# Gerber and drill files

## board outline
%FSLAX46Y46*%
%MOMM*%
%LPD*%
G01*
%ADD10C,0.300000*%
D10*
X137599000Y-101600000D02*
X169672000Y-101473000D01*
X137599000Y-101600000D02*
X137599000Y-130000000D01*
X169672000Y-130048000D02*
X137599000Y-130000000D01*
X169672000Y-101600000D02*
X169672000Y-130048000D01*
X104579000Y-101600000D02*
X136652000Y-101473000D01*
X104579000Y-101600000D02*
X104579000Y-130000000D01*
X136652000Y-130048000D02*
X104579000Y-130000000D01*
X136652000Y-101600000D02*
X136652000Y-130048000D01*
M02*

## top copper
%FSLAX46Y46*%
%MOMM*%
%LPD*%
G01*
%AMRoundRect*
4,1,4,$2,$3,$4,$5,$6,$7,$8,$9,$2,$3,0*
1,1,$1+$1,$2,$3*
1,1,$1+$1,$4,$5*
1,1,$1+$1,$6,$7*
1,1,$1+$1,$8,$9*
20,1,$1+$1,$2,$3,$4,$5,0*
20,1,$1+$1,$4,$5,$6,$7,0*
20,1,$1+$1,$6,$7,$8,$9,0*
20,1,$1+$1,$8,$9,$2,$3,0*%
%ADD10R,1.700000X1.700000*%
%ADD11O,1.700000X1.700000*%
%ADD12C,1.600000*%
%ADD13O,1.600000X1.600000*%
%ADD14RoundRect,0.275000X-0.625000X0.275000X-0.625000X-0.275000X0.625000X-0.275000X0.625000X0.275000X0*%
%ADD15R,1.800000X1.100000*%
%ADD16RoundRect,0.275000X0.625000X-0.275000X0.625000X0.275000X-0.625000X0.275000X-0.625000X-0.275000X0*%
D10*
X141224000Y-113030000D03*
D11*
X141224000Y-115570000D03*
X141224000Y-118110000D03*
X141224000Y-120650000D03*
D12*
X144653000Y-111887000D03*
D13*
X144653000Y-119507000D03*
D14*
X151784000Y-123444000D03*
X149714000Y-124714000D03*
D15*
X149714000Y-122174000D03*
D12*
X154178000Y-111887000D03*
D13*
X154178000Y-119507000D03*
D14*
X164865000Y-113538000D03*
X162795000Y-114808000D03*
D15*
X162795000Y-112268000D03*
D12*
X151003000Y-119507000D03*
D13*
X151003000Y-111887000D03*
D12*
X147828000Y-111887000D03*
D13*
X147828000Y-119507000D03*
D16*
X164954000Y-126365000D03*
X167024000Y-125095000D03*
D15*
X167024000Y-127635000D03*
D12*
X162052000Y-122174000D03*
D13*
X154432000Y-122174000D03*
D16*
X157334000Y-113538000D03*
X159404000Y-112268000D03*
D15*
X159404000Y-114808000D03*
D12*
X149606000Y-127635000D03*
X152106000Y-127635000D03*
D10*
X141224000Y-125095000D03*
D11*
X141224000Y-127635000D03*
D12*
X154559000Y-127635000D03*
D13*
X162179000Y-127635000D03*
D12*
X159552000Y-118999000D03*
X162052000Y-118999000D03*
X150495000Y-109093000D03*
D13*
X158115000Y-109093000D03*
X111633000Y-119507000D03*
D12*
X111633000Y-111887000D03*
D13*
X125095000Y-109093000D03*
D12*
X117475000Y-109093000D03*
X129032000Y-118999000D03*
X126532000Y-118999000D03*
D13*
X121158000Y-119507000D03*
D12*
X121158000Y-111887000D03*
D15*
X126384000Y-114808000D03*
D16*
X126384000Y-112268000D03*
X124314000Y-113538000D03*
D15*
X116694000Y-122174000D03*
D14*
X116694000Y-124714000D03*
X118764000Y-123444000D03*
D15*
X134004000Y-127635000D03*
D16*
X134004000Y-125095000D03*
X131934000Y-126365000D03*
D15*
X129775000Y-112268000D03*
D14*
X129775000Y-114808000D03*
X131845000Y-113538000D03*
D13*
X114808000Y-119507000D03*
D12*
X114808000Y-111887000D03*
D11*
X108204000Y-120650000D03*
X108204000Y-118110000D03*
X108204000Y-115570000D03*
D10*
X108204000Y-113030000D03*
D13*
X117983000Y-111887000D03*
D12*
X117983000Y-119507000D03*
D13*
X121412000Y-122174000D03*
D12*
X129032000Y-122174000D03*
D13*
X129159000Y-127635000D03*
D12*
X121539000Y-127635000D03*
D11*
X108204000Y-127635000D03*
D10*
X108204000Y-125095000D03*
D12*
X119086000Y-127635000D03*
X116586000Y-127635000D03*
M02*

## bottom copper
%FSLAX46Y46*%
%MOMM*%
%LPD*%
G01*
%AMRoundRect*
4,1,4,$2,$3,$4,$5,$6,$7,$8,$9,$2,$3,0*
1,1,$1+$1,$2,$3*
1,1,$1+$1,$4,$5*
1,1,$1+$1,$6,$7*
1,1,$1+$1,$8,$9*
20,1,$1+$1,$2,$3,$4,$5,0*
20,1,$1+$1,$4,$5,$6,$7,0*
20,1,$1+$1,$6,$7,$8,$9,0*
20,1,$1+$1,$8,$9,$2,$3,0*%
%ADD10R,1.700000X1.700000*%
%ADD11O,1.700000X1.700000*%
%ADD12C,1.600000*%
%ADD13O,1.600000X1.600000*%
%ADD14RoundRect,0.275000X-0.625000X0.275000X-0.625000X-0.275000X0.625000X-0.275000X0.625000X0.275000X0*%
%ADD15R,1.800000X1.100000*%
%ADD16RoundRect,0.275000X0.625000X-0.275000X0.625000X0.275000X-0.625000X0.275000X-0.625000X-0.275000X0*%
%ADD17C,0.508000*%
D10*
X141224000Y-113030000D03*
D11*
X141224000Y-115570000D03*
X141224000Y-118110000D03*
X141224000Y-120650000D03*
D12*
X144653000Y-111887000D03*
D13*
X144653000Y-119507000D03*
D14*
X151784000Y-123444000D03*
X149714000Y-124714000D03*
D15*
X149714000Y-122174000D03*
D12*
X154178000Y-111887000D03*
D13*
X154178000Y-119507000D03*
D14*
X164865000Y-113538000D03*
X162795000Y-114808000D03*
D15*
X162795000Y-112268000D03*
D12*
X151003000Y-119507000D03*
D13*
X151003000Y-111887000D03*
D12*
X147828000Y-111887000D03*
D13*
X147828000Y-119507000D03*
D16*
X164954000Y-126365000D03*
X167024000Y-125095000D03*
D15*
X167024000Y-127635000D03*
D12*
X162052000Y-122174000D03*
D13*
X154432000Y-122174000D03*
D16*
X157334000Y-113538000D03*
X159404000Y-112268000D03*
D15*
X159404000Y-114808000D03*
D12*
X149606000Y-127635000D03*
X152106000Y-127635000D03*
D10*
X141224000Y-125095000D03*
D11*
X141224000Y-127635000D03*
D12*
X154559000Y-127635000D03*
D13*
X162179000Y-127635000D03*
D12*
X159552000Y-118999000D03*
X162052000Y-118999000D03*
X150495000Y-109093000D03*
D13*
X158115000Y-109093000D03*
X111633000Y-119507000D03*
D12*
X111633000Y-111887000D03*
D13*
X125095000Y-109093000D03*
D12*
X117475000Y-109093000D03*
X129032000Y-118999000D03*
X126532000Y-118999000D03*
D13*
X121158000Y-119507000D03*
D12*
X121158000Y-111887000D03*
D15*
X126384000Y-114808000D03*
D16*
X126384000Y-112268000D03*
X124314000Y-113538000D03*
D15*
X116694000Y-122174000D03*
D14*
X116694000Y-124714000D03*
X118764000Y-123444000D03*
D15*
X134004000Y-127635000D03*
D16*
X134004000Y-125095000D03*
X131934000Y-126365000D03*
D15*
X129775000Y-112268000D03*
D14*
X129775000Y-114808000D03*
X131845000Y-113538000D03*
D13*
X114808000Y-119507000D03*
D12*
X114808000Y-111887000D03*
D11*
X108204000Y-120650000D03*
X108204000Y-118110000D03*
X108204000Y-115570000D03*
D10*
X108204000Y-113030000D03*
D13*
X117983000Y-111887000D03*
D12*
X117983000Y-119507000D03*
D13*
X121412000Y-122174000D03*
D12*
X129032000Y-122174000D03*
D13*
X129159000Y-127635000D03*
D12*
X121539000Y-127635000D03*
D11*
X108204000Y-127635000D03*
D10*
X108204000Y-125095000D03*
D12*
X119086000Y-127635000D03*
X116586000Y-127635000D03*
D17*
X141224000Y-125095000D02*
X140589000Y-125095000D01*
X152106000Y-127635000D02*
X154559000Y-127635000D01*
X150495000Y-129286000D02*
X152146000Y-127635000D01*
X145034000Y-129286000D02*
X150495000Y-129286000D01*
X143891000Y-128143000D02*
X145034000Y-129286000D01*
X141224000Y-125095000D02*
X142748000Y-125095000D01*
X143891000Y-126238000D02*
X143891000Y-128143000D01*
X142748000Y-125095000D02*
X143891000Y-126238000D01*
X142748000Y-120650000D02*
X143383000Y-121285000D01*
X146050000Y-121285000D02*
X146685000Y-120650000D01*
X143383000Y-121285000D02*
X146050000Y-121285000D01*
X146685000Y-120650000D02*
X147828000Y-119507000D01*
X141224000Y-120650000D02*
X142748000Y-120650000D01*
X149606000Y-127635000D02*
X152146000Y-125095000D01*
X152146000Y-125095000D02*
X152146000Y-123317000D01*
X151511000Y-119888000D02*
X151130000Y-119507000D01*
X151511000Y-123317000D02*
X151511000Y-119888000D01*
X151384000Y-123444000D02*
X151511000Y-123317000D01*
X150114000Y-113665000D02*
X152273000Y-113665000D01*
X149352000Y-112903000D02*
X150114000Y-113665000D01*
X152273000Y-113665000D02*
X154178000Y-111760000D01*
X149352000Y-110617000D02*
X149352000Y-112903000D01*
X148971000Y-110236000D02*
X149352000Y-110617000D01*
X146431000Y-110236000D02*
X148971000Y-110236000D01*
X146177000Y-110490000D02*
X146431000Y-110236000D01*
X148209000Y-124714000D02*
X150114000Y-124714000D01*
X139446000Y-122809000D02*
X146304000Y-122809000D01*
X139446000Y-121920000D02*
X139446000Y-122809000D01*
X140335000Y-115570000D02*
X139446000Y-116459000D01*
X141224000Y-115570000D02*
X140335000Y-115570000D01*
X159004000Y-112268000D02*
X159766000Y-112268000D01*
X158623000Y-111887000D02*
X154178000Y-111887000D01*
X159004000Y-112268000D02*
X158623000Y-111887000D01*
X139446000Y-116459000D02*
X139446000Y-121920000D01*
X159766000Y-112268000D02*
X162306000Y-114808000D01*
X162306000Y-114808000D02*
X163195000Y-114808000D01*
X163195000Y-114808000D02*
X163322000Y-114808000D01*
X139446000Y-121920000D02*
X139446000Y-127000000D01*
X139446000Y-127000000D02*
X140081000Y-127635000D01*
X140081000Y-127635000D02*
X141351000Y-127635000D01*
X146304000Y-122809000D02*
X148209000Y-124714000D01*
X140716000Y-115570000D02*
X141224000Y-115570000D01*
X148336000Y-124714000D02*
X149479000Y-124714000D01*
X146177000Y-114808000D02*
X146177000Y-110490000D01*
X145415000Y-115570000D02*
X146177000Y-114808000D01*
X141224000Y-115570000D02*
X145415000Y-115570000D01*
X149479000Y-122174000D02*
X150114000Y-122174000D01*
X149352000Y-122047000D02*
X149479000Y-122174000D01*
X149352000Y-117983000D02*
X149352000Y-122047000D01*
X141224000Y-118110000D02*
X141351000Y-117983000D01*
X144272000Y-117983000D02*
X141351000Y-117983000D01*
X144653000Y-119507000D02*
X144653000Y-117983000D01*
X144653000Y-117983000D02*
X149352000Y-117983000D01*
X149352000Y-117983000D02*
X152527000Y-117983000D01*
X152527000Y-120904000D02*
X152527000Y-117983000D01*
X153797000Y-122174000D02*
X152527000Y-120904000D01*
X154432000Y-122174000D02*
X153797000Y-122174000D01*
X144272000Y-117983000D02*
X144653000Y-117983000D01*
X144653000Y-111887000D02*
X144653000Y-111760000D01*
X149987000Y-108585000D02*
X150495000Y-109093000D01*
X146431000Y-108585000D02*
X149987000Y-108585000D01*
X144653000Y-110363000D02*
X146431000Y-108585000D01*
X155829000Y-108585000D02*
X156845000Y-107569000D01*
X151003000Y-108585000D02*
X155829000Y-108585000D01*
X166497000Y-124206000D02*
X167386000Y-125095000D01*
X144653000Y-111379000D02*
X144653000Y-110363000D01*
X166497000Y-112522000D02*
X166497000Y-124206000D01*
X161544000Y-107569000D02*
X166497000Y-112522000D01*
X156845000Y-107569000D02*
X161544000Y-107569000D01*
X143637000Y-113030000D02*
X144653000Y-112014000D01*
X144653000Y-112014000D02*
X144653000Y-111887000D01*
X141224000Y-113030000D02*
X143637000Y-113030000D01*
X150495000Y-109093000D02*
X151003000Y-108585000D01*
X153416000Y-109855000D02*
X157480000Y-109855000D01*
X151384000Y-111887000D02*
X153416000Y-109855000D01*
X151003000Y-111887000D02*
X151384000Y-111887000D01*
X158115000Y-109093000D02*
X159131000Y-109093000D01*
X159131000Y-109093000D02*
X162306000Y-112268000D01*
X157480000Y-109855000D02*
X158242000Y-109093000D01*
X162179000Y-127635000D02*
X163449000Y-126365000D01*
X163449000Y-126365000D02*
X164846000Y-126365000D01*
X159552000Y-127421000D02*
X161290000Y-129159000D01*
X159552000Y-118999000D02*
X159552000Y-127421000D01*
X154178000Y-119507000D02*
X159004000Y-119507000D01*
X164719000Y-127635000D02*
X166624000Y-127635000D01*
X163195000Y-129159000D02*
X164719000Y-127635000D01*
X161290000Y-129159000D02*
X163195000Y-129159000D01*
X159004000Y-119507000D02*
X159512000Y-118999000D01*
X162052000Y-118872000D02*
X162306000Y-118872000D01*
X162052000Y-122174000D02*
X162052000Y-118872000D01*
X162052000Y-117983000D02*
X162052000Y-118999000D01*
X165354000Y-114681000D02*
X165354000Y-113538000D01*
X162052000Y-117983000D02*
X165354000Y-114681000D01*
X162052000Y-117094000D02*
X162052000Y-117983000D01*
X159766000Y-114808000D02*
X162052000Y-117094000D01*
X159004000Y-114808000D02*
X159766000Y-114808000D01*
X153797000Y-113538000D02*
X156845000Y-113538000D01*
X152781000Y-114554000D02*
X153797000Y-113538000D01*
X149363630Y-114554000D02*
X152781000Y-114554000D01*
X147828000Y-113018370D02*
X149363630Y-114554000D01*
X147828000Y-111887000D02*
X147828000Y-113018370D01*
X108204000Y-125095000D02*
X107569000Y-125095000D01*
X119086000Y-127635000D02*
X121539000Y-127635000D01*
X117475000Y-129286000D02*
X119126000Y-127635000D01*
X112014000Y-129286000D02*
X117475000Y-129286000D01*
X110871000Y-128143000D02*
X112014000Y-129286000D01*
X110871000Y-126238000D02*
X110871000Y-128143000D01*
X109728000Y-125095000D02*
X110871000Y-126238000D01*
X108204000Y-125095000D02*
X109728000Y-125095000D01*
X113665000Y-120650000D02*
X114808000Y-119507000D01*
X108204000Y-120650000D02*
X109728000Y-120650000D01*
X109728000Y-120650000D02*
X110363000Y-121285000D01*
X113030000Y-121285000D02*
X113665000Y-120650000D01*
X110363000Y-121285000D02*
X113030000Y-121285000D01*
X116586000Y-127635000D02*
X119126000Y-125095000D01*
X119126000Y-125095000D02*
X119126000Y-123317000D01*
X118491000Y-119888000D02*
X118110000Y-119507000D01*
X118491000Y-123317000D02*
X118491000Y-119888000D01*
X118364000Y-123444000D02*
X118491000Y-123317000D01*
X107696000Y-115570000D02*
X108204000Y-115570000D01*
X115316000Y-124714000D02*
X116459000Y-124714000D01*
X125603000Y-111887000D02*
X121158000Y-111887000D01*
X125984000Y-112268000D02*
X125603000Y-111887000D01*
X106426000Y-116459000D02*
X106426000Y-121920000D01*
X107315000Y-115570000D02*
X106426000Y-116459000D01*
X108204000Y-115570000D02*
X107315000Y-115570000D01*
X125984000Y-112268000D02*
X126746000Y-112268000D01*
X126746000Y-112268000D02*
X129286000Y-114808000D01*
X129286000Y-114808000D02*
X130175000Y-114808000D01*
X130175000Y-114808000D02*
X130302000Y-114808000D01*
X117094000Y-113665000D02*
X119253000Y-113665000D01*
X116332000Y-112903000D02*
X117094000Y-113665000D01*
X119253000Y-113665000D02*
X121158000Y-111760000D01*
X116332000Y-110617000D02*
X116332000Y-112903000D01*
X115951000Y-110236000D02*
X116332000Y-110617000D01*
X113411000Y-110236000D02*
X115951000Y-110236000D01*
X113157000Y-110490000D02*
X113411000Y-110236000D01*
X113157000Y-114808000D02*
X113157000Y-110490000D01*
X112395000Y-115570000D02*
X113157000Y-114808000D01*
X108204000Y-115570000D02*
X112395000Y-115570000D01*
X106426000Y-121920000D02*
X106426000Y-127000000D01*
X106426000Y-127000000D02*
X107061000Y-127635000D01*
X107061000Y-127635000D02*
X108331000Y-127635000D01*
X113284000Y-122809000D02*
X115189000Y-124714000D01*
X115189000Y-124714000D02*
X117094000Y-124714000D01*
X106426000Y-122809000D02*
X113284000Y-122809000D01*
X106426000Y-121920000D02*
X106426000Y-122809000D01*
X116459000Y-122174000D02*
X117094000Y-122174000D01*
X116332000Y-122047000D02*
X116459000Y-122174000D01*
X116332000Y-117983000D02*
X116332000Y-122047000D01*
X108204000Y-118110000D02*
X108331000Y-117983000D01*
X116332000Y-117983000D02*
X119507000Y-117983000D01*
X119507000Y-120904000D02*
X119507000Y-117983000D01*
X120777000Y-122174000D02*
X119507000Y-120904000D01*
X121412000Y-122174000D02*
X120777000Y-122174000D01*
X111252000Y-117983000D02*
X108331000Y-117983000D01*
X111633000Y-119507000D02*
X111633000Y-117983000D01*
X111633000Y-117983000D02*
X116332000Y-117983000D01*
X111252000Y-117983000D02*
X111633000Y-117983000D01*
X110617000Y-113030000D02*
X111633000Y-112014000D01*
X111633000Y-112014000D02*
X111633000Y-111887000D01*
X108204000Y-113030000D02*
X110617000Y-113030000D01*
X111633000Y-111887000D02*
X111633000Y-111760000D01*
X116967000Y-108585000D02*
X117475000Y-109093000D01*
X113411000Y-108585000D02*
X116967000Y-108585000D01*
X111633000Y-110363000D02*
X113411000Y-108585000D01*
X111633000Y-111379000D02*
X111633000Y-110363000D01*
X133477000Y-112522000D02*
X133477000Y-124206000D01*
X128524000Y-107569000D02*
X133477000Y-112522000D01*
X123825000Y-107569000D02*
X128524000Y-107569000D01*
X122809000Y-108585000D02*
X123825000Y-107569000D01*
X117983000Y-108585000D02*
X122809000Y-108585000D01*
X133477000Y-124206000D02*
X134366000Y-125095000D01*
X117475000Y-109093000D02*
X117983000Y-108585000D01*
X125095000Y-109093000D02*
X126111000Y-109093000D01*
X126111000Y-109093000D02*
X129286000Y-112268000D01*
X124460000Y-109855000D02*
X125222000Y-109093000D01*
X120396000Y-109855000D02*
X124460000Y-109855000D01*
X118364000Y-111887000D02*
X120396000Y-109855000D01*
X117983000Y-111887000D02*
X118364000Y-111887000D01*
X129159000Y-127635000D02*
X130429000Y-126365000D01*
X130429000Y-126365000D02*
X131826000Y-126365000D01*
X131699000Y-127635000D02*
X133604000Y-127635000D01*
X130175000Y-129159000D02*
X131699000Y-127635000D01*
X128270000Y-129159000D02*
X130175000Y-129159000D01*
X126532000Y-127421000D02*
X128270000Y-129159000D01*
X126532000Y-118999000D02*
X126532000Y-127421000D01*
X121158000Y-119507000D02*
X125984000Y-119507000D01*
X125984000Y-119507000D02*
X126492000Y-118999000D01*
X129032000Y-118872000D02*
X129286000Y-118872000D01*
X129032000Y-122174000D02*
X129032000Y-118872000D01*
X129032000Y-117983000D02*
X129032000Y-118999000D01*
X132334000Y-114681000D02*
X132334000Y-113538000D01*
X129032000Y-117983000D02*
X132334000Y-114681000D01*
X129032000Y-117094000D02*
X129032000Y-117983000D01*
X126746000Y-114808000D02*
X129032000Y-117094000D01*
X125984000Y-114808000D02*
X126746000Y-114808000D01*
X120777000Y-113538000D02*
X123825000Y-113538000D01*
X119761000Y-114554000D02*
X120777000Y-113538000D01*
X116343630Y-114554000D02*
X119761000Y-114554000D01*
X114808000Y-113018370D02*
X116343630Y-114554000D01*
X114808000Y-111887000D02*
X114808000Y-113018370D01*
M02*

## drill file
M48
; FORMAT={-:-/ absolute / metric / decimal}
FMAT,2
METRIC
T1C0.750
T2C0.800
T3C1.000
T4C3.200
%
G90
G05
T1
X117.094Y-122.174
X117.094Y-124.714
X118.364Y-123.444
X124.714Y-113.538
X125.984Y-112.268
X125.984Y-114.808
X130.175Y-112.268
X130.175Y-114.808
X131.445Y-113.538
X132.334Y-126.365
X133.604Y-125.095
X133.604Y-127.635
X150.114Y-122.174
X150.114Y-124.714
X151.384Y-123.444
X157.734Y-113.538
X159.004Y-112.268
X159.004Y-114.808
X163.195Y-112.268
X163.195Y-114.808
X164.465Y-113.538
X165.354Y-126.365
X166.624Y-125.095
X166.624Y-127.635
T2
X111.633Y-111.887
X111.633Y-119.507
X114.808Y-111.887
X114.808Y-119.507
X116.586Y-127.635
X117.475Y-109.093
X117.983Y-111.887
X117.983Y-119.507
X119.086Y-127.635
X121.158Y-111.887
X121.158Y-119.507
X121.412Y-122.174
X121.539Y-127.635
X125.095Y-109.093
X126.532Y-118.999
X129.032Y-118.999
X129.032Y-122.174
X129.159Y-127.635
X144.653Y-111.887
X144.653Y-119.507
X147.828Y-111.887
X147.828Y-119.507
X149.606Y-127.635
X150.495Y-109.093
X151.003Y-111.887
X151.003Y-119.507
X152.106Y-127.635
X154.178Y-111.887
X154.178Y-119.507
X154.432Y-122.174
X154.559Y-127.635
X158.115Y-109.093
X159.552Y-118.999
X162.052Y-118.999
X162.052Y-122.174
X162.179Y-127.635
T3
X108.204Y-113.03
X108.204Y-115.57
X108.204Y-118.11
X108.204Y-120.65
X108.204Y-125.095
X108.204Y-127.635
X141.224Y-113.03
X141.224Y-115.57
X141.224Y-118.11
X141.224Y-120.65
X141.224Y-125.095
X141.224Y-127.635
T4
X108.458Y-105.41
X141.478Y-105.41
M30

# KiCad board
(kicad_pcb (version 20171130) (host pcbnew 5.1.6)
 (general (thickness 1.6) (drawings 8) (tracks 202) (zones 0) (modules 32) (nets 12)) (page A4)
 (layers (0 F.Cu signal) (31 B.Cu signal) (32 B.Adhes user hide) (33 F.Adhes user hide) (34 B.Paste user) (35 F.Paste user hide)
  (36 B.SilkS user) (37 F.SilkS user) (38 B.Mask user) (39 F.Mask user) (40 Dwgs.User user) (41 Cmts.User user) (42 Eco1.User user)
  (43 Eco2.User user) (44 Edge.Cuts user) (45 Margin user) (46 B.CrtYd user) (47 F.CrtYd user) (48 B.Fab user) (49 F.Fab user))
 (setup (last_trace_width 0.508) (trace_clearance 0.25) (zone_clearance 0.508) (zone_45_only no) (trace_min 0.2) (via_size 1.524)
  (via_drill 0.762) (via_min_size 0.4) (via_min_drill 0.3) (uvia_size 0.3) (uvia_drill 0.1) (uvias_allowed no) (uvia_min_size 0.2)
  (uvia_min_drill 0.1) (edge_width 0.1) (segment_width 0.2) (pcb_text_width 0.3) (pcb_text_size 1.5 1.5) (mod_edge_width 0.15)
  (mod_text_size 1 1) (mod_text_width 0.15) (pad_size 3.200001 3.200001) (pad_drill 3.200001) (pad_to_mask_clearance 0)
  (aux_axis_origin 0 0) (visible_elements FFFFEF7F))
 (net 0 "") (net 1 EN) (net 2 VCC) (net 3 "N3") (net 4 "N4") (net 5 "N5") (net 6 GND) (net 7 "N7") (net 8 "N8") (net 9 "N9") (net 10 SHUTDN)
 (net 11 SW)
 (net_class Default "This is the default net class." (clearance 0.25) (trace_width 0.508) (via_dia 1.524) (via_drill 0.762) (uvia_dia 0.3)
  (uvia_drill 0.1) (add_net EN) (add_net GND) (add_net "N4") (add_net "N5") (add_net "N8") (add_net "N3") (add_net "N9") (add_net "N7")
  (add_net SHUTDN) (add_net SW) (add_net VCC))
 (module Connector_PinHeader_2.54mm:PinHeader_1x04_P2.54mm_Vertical (layer F.Cu) (at 141.224 113.03)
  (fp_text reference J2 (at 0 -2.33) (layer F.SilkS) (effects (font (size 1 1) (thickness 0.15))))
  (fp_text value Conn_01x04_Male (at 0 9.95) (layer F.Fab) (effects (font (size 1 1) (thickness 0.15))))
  (pad 1 thru_hole rect (at 0 0) (size 1.7 1.7) (drill 1) (layers *.Cu *.Mask))
  (pad 2 thru_hole oval (at 0 2.54) (size 1.7 1.7) (drill 1) (layers *.Cu *.Mask))
  (pad 3 thru_hole oval (at 0 5.08) (size 1.7 1.7) (drill 1) (layers *.Cu *.Mask))
  (pad 4 thru_hole oval (at 0 7.62) (size 1.7 1.7) (drill 1) (layers *.Cu *.Mask)))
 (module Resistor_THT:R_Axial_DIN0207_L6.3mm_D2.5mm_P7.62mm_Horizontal (layer F.Cu) (at 144.653 111.887 270)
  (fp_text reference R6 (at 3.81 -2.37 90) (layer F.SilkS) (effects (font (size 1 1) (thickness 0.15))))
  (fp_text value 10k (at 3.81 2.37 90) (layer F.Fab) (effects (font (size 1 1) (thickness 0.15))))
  (pad 1 thru_hole circle (at 0 0 270) (size 1.6 1.6) (drill 0.8) (layers *.Cu *.Mask))
  (pad 2 thru_hole oval (at 7.62 0 270) (size 1.6 1.6) (drill 0.8) (layers *.Cu *.Mask)))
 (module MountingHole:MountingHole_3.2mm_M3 (layer F.Cu) (at 141.478 105.41)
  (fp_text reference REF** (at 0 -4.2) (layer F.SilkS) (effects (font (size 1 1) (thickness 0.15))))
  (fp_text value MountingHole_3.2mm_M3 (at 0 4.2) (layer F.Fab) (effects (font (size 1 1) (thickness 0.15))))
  (pad "" np_thru_hole circle (at 0 0) (size 3.200001 3.200001) (drill 3.200001) (layers *.Cu *.Mask)))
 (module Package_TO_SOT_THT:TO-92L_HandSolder (layer F.Cu) (at 150.114 122.174 270)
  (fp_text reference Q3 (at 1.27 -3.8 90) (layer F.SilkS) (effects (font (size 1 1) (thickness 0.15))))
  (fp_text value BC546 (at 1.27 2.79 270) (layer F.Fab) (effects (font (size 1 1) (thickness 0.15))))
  (pad 2 thru_hole roundrect (at 1.27 -1.27 270) (size 1.1 1.8) (drill 0.75 (offset 0 -0.4)) (layers *.Cu *.Mask) (roundrect_rratio 0.25))
  (pad 3 thru_hole roundrect (at 2.54 0 270) (size 1.1 1.8) (drill 0.75 (offset 0 0.4)) (layers *.Cu *.Mask) (roundrect_rratio 0.25))
  (pad 1 thru_hole rect (at 0 0 270) (size 1.1 1.8) (drill 0.75 (offset 0 0.4)) (layers *.Cu *.Mask)))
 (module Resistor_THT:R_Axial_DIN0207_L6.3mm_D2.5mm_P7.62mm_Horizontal (layer F.Cu) (at 154.178 111.887 270)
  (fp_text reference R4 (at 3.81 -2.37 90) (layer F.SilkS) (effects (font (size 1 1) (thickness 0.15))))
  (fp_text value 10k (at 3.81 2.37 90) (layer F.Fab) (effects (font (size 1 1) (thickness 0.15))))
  (pad 1 thru_hole circle (at 0 0 270) (size 1.6 1.6) (drill 0.8) (layers *.Cu *.Mask))
  (pad 2 thru_hole oval (at 7.62 0 270) (size 1.6 1.6) (drill 0.8) (layers *.Cu *.Mask)))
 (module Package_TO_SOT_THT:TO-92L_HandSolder (layer F.Cu) (at 163.195 112.268 270)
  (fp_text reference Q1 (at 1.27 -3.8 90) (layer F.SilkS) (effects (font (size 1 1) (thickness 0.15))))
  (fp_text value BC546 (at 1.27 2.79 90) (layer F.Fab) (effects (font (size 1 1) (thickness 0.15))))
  (pad 2 thru_hole roundrect (at 1.27 -1.27 270) (size 1.1 1.8) (drill 0.75 (offset 0 -0.4)) (layers *.Cu *.Mask) (roundrect_rratio 0.25))
  (pad 3 thru_hole roundrect (at 2.54 0 270) (size 1.1 1.8) (drill 0.75 (offset 0 0.4)) (layers *.Cu *.Mask) (roundrect_rratio 0.25))
  (pad 1 thru_hole rect (at 0 0 270) (size 1.1 1.8) (drill 0.75 (offset 0 0.4)) (layers *.Cu *.Mask)))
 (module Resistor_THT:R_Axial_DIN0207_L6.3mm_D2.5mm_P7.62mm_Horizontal (layer F.Cu) (at 151.003 119.507 90)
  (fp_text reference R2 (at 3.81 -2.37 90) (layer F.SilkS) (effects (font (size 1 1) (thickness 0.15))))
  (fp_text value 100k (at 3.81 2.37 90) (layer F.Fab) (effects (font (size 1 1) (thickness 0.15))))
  (pad 1 thru_hole circle (at 0 0 90) (size 1.6 1.6) (drill 0.8) (layers *.Cu *.Mask))
  (pad 2 thru_hole oval (at 7.62 0 90) (size 1.6 1.6) (drill 0.8) (layers *.Cu *.Mask)))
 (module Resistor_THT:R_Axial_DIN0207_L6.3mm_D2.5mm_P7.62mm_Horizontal (layer F.Cu) (at 147.828 111.887 270)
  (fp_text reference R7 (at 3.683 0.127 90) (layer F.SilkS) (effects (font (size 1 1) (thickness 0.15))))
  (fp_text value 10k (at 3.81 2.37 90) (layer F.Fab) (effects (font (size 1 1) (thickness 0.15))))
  (pad 1 thru_hole circle (at 0 0 270) (size 1.6 1.6) (drill 0.8) (layers *.Cu *.Mask))
  (pad 2 thru_hole oval (at 7.62 0 270) (size 1.6 1.6) (drill 0.8) (layers *.Cu *.Mask)))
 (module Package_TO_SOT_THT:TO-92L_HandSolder (layer F.Cu) (at 166.624 127.635 90)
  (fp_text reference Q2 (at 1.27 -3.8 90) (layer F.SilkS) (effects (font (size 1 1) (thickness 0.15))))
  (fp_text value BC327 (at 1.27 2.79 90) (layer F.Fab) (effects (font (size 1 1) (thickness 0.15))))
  (pad 2 thru_hole roundrect (at 1.27 -1.27 90) (size 1.1 1.8) (drill 0.75 (offset 0 -0.4)) (layers *.Cu *.Mask) (roundrect_rratio 0.25))
  (pad 3 thru_hole roundrect (at 2.54 0 90) (size 1.1 1.8) (drill 0.75 (offset 0 0.4)) (layers *.Cu *.Mask) (roundrect_rratio 0.25))
  (pad 1 thru_hole rect (at 0 0 90) (size 1.1 1.8) (drill 0.75 (offset 0 0.4)) (layers *.Cu *.Mask)))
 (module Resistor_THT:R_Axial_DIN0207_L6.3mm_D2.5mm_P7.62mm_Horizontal (layer F.Cu) (at 162.052 122.174 180)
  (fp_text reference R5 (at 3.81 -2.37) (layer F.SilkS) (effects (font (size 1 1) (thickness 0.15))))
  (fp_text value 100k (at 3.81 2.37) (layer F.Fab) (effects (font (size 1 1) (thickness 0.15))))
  (pad 1 thru_hole circle (at 0 0 180) (size 1.6 1.6) (drill 0.8) (layers *.Cu *.Mask))
  (pad 2 thru_hole oval (at 7.62 0 180) (size 1.6 1.6) (drill 0.8) (layers *.Cu *.Mask)))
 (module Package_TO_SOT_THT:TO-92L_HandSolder (layer F.Cu) (at 159.004 114.808 90)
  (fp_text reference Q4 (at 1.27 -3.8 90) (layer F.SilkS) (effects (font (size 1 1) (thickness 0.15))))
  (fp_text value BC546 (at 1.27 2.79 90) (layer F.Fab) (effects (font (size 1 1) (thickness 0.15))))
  (pad 2 thru_hole roundrect (at 1.27 -1.27 90) (size 1.1 1.8) (drill 0.75 (offset 0 -0.4)) (layers *.Cu *.Mask) (roundrect_rratio 0.25))
  (pad 3 thru_hole roundrect (at 2.54 0 90) (size 1.1 1.8) (drill 0.75 (offset 0 0.4)) (layers *.Cu *.Mask) (roundrect_rratio 0.25))
  (pad 1 thru_hole rect (at 0 0 90) (size 1.1 1.8) (drill 0.75 (offset 0 0.4)) (layers *.Cu *.Mask)))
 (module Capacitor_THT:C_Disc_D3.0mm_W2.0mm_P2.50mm (layer F.Cu) (at 149.606 127.635)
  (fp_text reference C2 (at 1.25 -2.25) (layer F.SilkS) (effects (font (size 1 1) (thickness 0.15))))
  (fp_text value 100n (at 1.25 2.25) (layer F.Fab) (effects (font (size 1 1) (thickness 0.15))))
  (pad 1 thru_hole circle (at 0 0) (size 1.6 1.6) (drill 0.8) (layers *.Cu *.Mask))
  (pad 2 thru_hole circle (at 2.5 0) (size 1.6 1.6) (drill 0.8) (layers *.Cu *.Mask)))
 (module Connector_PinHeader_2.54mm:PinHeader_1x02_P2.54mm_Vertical (layer F.Cu) (at 141.224 125.095)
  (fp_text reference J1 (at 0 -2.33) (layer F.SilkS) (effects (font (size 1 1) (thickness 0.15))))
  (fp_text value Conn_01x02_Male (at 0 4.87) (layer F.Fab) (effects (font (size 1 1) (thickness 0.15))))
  (pad 1 thru_hole rect (at 0 0) (size 1.7 1.7) (drill 1) (layers *.Cu *.Mask))
  (pad 2 thru_hole oval (at 0 2.54) (size 1.7 1.7) (drill 1) (layers *.Cu *.Mask)))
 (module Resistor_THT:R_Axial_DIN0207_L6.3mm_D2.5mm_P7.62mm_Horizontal (layer F.Cu) (at 154.559 127.635)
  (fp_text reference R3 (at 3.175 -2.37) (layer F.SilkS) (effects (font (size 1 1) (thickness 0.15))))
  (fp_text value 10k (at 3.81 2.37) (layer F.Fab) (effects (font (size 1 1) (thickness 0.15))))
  (pad 1 thru_hole circle (at 0 0) (size 1.6 1.6) (drill 0.8) (layers *.Cu *.Mask))
  (pad 2 thru_hole oval (at 7.62 0) (size 1.6 1.6) (drill 0.8) (layers *.Cu *.Mask)))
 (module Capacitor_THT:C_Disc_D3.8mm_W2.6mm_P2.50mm (layer F.Cu) (at 162.052 118.999 180)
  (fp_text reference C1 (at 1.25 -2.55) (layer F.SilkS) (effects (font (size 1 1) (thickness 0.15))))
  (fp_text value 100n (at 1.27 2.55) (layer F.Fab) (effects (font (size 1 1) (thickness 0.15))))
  (pad 2 thru_hole circle (at 2.5 0 180) (size 1.6 1.6) (drill 0.8) (layers *.Cu *.Mask))
  (pad 1 thru_hole circle (at 0 0 180) (size 1.6 1.6) (drill 0.8) (layers *.Cu *.Mask)))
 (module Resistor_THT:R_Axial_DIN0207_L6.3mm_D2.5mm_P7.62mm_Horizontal (layer F.Cu) (at 150.495 109.093)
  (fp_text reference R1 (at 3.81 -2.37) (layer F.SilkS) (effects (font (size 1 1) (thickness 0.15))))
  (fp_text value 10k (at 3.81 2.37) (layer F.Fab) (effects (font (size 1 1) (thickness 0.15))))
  (pad 1 thru_hole circle (at 0 0) (size 1.6 1.6) (drill 0.8) (layers *.Cu *.Mask))
  (pad 2 thru_hole oval (at 7.62 0) (size 1.6 1.6) (drill 0.8) (layers *.Cu *.Mask)))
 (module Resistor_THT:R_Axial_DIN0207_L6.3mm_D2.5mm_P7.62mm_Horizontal (layer F.Cu) (at 111.633 111.887 270)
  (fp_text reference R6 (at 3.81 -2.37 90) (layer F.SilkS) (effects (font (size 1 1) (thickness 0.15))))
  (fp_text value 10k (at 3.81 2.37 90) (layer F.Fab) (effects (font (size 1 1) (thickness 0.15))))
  (pad 2 thru_hole oval (at 7.62 0 270) (size 1.6 1.6) (drill 0.8) (layers *.Cu *.Mask) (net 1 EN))
  (pad 1 thru_hole circle (at 0 0 270) (size 1.6 1.6) (drill 0.8) (layers *.Cu *.Mask) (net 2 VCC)))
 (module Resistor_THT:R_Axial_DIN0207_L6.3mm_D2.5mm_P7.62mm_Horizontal (layer F.Cu) (at 117.475 109.093)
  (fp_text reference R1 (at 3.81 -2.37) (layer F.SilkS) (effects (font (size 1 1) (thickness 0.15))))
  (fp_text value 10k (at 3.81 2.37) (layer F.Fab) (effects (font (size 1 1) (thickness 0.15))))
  (pad 2 thru_hole oval (at 7.62 0) (size 1.6 1.6) (drill 0.8) (layers *.Cu *.Mask) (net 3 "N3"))
  (pad 1 thru_hole circle (at 0 0) (size 1.6 1.6) (drill 0.8) (layers *.Cu *.Mask) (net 2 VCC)))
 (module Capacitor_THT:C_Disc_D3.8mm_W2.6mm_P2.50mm (layer F.Cu) (at 129.032 118.999 180)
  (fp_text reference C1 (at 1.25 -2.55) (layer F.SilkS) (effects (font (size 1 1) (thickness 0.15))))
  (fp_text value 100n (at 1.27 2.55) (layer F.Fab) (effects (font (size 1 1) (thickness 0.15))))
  (pad 1 thru_hole circle (at 0 0 180) (size 1.6 1.6) (drill 0.8) (layers *.Cu *.Mask) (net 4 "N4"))
  (pad 2 thru_hole circle (at 2.5 0 180) (size 1.6 1.6) (drill 0.8) (layers *.Cu *.Mask) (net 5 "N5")))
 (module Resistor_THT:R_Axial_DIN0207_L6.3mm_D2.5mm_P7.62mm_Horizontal (layer F.Cu) (at 121.158 111.887 270)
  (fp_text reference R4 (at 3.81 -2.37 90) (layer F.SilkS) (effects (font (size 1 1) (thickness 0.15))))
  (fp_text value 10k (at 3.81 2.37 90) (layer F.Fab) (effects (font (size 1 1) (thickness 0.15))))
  (pad 2 thru_hole oval (at 7.62 0 270) (size 1.6 1.6) (drill 0.8) (layers *.Cu *.Mask) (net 5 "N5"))
  (pad 1 thru_hole circle (at 0 0 270) (size 1.6 1.6) (drill 0.8) (layers *.Cu *.Mask) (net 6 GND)))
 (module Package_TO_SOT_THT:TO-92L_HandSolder (layer F.Cu) (at 125.984 114.808 90)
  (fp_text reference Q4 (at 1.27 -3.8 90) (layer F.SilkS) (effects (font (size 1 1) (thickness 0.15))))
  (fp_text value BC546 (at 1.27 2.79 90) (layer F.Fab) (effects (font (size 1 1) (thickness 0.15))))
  (pad 1 thru_hole rect (at 0 0 90) (size 1.1 1.8) (drill 0.75 (offset 0 0.4)) (layers *.Cu *.Mask) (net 4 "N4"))
  (pad 3 thru_hole roundrect (at 2.54 0 90) (size 1.1 1.8) (drill 0.75 (offset 0 0.4)) (layers *.Cu *.Mask) (roundrect_rratio 0.25)
   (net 6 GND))
  (pad 2 thru_hole roundrect (at 1.27 -1.27 90) (size 1.1 1.8) (drill 0.75 (offset 0 -0.4)) (layers *.Cu *.Mask) (roundrect_rratio 0.25)
   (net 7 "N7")))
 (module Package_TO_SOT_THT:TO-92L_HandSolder (layer F.Cu) (at 117.094 122.174 270)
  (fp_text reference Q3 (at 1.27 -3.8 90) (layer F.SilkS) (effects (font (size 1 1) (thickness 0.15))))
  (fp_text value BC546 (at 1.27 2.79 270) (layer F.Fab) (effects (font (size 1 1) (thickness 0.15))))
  (pad 1 thru_hole rect (at 0 0 270) (size 1.1 1.8) (drill 0.75 (offset 0 0.4)) (layers *.Cu *.Mask) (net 1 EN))
  (pad 3 thru_hole roundrect (at 2.54 0 270) (size 1.1 1.8) (drill 0.75 (offset 0 0.4)) (layers *.Cu *.Mask) (roundrect_rratio 0.25)
   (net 6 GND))
  (pad 2 thru_hole roundrect (at 1.27 -1.27 270) (size 1.1 1.8) (drill 0.75 (offset 0 -0.4)) (layers *.Cu *.Mask) (roundrect_rratio 0.25)
   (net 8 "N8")))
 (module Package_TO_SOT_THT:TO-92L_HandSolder (layer F.Cu) (at 133.604 127.635 90)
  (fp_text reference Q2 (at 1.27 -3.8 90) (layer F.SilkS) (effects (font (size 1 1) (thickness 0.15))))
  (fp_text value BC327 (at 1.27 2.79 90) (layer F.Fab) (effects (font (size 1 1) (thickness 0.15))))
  (pad 1 thru_hole rect (at 0 0 90) (size 1.1 1.8) (drill 0.75 (offset 0 0.4)) (layers *.Cu *.Mask) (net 5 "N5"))
  (pad 3 thru_hole roundrect (at 2.54 0 90) (size 1.1 1.8) (drill 0.75 (offset 0 0.4)) (layers *.Cu *.Mask) (roundrect_rratio 0.25)
   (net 2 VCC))
  (pad 2 thru_hole roundrect (at 1.27 -1.27 90) (size 1.1 1.8) (drill 0.75 (offset 0 -0.4)) (layers *.Cu *.Mask) (roundrect_rratio 0.25)
   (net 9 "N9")))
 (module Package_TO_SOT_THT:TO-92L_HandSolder (layer F.Cu) (at 130.175 112.268 270)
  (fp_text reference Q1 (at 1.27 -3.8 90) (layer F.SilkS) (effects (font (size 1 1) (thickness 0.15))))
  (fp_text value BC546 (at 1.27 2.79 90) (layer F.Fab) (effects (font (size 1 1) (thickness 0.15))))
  (pad 1 thru_hole rect (at 0 0 270) (size 1.1 1.8) (drill 0.75 (offset 0 0.4)) (layers *.Cu *.Mask) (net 3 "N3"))
  (pad 3 thru_hole roundrect (at 2.54 0 270) (size 1.1 1.8) (drill 0.75 (offset 0 0.4)) (layers *.Cu *.Mask) (roundrect_rratio 0.25)
   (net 6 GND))
  (pad 2 thru_hole roundrect (at 1.27 -1.27 270) (size 1.1 1.8) (drill 0.75 (offset 0 -0.4)) (layers *.Cu *.Mask) (roundrect_rratio 0.25)
   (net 4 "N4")))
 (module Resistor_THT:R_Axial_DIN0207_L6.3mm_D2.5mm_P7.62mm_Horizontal (layer F.Cu) (at 114.808 111.887 270)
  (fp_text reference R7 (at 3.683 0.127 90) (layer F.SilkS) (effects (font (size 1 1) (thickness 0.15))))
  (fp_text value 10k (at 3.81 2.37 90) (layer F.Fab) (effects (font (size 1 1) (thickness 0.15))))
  (pad 2 thru_hole oval (at 7.62 0 270) (size 1.6 1.6) (drill 0.8) (layers *.Cu *.Mask) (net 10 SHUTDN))
  (pad 1 thru_hole circle (at 0 0 270) (size 1.6 1.6) (drill 0.8) (layers *.Cu *.Mask) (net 7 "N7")))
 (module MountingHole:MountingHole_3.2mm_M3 (layer F.Cu) (at 108.458 105.41)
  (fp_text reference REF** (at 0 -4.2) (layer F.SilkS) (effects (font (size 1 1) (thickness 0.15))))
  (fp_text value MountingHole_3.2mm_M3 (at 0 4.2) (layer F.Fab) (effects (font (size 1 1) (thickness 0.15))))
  (pad "" np_thru_hole circle (at 0 0) (size 3.200001 3.200001) (drill 3.200001) (layers *.Cu *.Mask)))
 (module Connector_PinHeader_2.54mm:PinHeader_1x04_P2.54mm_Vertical (layer F.Cu) (at 108.204 113.03)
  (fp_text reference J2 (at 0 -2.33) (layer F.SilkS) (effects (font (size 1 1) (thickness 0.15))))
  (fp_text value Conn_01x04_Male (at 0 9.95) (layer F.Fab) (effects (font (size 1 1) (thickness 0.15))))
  (pad 4 thru_hole oval (at 0 7.62) (size 1.7 1.7) (drill 1) (layers *.Cu *.Mask) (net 10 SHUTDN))
  (pad 3 thru_hole oval (at 0 5.08) (size 1.7 1.7) (drill 1) (layers *.Cu *.Mask) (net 1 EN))
  (pad 2 thru_hole oval (at 0 2.54) (size 1.7 1.7) (drill 1) (layers *.Cu *.Mask) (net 6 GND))
  (pad 1 thru_hole rect (at 0 0) (size 1.7 1.7) (drill 1) (layers *.Cu *.Mask) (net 2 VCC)))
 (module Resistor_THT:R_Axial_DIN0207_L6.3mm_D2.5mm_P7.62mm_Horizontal (layer F.Cu) (at 117.983 119.507 90)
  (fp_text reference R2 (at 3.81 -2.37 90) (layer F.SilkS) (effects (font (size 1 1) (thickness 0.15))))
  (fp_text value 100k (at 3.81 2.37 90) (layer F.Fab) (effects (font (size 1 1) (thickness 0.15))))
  (pad 2 thru_hole oval (at 7.62 0 90) (size 1.6 1.6) (drill 0.8) (layers *.Cu *.Mask) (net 3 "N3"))
  (pad 1 thru_hole circle (at 0 0 90) (size 1.6 1.6) (drill 0.8) (layers *.Cu *.Mask) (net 8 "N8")))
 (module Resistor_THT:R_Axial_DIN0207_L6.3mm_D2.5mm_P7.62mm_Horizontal (layer F.Cu) (at 129.032 122.174 180)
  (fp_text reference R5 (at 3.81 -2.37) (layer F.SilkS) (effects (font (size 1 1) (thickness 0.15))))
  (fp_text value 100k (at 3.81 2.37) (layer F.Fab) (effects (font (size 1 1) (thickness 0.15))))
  (pad 2 thru_hole oval (at 7.62 0 180) (size 1.6 1.6) (drill 0.8) (layers *.Cu *.Mask) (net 1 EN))
  (pad 1 thru_hole circle (at 0 0 180) (size 1.6 1.6) (drill 0.8) (layers *.Cu *.Mask) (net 4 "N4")))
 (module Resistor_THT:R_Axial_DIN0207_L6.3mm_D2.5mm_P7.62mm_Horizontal (layer F.Cu) (at 121.539 127.635)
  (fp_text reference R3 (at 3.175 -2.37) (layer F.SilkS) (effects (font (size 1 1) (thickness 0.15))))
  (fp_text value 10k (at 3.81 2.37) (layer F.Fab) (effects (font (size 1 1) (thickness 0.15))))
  (pad 2 thru_hole oval (at 7.62 0) (size 1.6 1.6) (drill 0.8) (layers *.Cu *.Mask) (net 9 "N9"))
  (pad 1 thru_hole circle (at 0 0) (size 1.6 1.6) (drill 0.8) (layers *.Cu *.Mask) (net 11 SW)))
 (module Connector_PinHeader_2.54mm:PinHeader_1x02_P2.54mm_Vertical (layer F.Cu) (at 108.204 125.095)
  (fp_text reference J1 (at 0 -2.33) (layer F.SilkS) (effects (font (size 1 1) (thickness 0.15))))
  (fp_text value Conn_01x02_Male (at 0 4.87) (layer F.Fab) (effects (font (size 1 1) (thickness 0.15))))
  (pad 2 thru_hole oval (at 0 2.54) (size 1.7 1.7) (drill 1) (layers *.Cu *.Mask) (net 6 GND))
  (pad 1 thru_hole rect (at 0 0) (size 1.7 1.7) (drill 1) (layers *.Cu *.Mask) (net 11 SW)))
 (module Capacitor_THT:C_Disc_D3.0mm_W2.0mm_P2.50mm (layer F.Cu) (at 116.586 127.635)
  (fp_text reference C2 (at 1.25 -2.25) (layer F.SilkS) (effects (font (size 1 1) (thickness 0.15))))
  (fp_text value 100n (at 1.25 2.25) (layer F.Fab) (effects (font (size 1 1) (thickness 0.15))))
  (pad 2 thru_hole circle (at 2.5 0) (size 1.6 1.6) (drill 0.8) (layers *.Cu *.Mask) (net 11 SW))
  (pad 1 thru_hole circle (at 0 0) (size 1.6 1.6) (drill 0.8) (layers *.Cu *.Mask) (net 8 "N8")))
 (gr_line (start 137.599 101.6) (end 169.672 101.473) (layer Edge.Cuts) (width 0.3))
 (gr_line (start 137.599 101.6) (end 137.599 130) (layer Edge.Cuts) (width 0.3))
 (gr_line (start 169.672 130.048) (end 137.599 130) (layer Edge.Cuts) (width 0.3))
 (gr_line (start 169.672 101.6) (end 169.672 130.048) (layer Edge.Cuts) (width 0.3))
 (gr_line (start 104.579 101.6) (end 136.652 101.473) (layer Edge.Cuts) (width 0.3))
 (gr_line (start 104.579 101.6) (end 104.579 130) (layer Edge.Cuts) (width 0.3))
 (gr_line (start 136.652 130.048) (end 104.579 130) (layer Edge.Cuts) (width 0.3))
 (gr_line (start 136.652 101.6) (end 136.652 130.048) (layer Edge.Cuts) (width 0.3))
 (segment (start 141.224 125.095) (end 140.589 125.095) (width 0.508) (layer B.Cu) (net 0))
 (segment (start 152.106 127.635) (end 154.559 127.635) (width 0.508) (layer B.Cu) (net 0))
 (segment (start 150.495 129.286) (end 152.146 127.635) (width 0.508) (layer B.Cu) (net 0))
 (segment (start 145.034 129.286) (end 150.495 129.286) (width 0.508) (layer B.Cu) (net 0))
 (segment (start 143.891 128.143) (end 145.034 129.286) (width 0.508) (layer B.Cu) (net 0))
 (segment (start 141.224 125.095) (end 142.748 125.095) (width 0.508) (layer B.Cu) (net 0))
 (segment (start 143.891 126.238) (end 143.891 128.143) (width 0.508) (layer B.Cu) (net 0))
 (segment (start 142.748 125.095) (end 143.891 126.238) (width 0.508) (layer B.Cu) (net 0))
 (segment (start 142.748 120.65) (end 143.383 121.285) (width 0.508) (layer B.Cu) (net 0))
 (segment (start 146.05 121.285) (end 146.685 120.65) (width 0.508) (layer B.Cu) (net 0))
 (segment (start 143.383 121.285) (end 146.05 121.285) (width 0.508) (layer B.Cu) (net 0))
 (segment (start 146.685 120.65) (end 147.828 119.507) (width 0.508) (layer B.Cu) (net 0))
 (segment (start 141.224 120.65) (end 142.748 120.65) (width 0.508) (layer B.Cu) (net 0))
 (segment (start 149.606 127.635) (end 152.146 125.095) (width 0.508) (layer B.Cu) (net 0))
 (segment (start 152.146 125.095) (end 152.146 123.317) (width 0.508) (layer B.Cu) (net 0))
 (segment (start 151.511 119.888) (end 151.13 119.507) (width 0.508) (layer B.Cu) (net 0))
 (segment (start 151.511 123.317) (end 151.511 119.888) (width 0.508) (layer B.Cu) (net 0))
 (segment (start 151.384 123.444) (end 151.511 123.317) (width 0.508) (layer B.Cu) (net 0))
 (segment (start 150.114 113.665) (end 152.273 113.665) (width 0.508) (layer B.Cu) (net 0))
 (segment (start 149.352 112.903) (end 150.114 113.665) (width 0.508) (layer B.Cu) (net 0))
 (segment (start 152.273 113.665) (end 154.178 111.76) (width 0.508) (layer B.Cu) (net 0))
 (segment (start 149.352 110.617) (end 149.352 112.903) (width 0.508) (layer B.Cu) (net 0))
 (segment (start 148.971 110.236) (end 149.352 110.617) (width 0.508) (layer B.Cu) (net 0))
 (segment (start 146.431 110.236) (end 148.971 110.236) (width 0.508) (layer B.Cu) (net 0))
 (segment (start 146.177 110.49) (end 146.431 110.236) (width 0.508) (layer B.Cu) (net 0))
 (segment (start 148.209 124.714) (end 150.114 124.714) (width 0.508) (layer B.Cu) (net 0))
 (segment (start 139.446 122.809) (end 146.304 122.809) (width 0.508) (layer B.Cu) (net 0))
 (segment (start 139.446 121.92) (end 139.446 122.809) (width 0.508) (layer B.Cu) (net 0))
 (segment (start 140.335 115.57) (end 139.446 116.459) (width 0.508) (layer B.Cu) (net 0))
 (segment (start 141.224 115.57) (end 140.335 115.57) (width 0.508) (layer B.Cu) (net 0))
 (segment (start 159.004 112.268) (end 159.766 112.268) (width 0.508) (layer B.Cu) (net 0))
 (segment (start 158.623 111.887) (end 154.178 111.887) (width 0.508) (layer B.Cu) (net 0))
 (segment (start 159.004 112.268) (end 158.623 111.887) (width 0.508) (layer B.Cu) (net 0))
 (segment (start 139.446 116.459) (end 139.446 121.92) (width 0.508) (layer B.Cu) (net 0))
 (segment (start 159.766 112.268) (end 162.306 114.808) (width 0.508) (layer B.Cu) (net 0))
 (segment (start 162.306 114.808) (end 163.195 114.808) (width 0.508) (layer B.Cu) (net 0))
 (segment (start 163.195 114.808) (end 163.322 114.808) (width 0.508) (layer B.Cu) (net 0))
 (segment (start 139.446 121.92) (end 139.446 127) (width 0.508) (layer B.Cu) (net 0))
 (segment (start 139.446 127) (end 140.081 127.635) (width 0.508) (layer B.Cu) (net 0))
 (segment (start 140.081 127.635) (end 141.351 127.635) (width 0.508) (layer B.Cu) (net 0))
 (segment (start 146.304 122.809) (end 148.209 124.714) (width 0.508) (layer B.Cu) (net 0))
 (segment (start 140.716 115.57) (end 141.224 115.57) (width 0.508) (layer B.Cu) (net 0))
 (segment (start 148.336 124.714) (end 149.479 124.714) (width 0.508) (layer B.Cu) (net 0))
 (segment (start 146.177 114.808) (end 146.177 110.49) (width 0.508) (layer B.Cu) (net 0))
 (segment (start 145.415 115.57) (end 146.177 114.808) (width 0.508) (layer B.Cu) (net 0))
 (segment (start 141.224 115.57) (end 145.415 115.57) (width 0.508) (layer B.Cu) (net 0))
 (segment (start 149.479 122.174) (end 150.114 122.174) (width 0.508) (layer B.Cu) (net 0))
 (segment (start 149.352 122.047) (end 149.479 122.174) (width 0.508) (layer B.Cu) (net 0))
 (segment (start 149.352 117.983) (end 149.352 122.047) (width 0.508) (layer B.Cu) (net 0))
 (segment (start 141.224 118.11) (end 141.351 117.983) (width 0.508) (layer B.Cu) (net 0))
 (segment (start 144.272 117.983) (end 141.351 117.983) (width 0.508) (layer B.Cu) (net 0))
 (segment (start 144.653 119.507) (end 144.653 117.983) (width 0.508) (layer B.Cu) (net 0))
 (segment (start 144.653 117.983) (end 149.352 117.983) (width 0.508) (layer B.Cu) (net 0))
 (segment (start 149.352 117.983) (end 152.527 117.983) (width 0.508) (layer B.Cu) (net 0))
 (segment (start 152.527 120.904) (end 152.527 117.983) (width 0.508) (layer B.Cu) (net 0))
 (segment (start 153.797 122.174) (end 152.527 120.904) (width 0.508) (layer B.Cu) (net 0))
 (segment (start 154.432 122.174) (end 153.797 122.174) (width 0.508) (layer B.Cu) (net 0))
 (segment (start 144.272 117.983) (end 144.653 117.983) (width 0.508) (layer B.Cu) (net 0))
 (segment (start 144.653 111.887) (end 144.653 111.76) (width 0.508) (layer B.Cu) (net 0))
 (segment (start 149.987 108.585) (end 150.495 109.093) (width 0.508) (layer B.Cu) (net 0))
 (segment (start 146.431 108.585) (end 149.987 108.585) (width 0.508) (layer B.Cu) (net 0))
 (segment (start 144.653 110.363) (end 146.431 108.585) (width 0.508) (layer B.Cu) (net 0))
 (segment (start 155.829 108.585) (end 156.845 107.569) (width 0.508) (layer B.Cu) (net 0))
 (segment (start 151.003 108.585) (end 155.829 108.585) (width 0.508) (layer B.Cu) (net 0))
 (segment (start 166.497 124.206) (end 167.386 125.095) (width 0.508) (layer B.Cu) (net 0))
 (segment (start 144.653 111.379) (end 144.653 110.363) (width 0.508) (layer B.Cu) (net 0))
 (segment (start 166.497 112.522) (end 166.497 124.206) (width 0.508) (layer B.Cu) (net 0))
 (segment (start 161.544 107.569) (end 166.497 112.522) (width 0.508) (layer B.Cu) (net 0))
 (segment (start 156.845 107.569) (end 161.544 107.569) (width 0.508) (layer B.Cu) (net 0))
 (segment (start 143.637 113.03) (end 144.653 112.014) (width 0.508) (layer B.Cu) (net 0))
 (segment (start 144.653 112.014) (end 144.653 111.887) (width 0.508) (layer B.Cu) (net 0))
 (segment (start 141.224 113.03) (end 143.637 113.03) (width 0.508) (layer B.Cu) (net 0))
 (segment (start 150.495 109.093) (end 151.003 108.585) (width 0.508) (layer B.Cu) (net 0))
 (segment (start 153.416 109.855) (end 157.48 109.855) (width 0.508) (layer B.Cu) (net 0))
 (segment (start 151.384 111.887) (end 153.416 109.855) (width 0.508) (layer B.Cu) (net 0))
 (segment (start 151.003 111.887) (end 151.384 111.887) (width 0.508) (layer B.Cu) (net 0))
 (segment (start 158.115 109.093) (end 159.131 109.093) (width 0.508) (layer B.Cu) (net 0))
 (segment (start 159.131 109.093) (end 162.306 112.268) (width 0.508) (layer B.Cu) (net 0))
 (segment (start 157.48 109.855) (end 158.242 109.093) (width 0.508) (layer B.Cu) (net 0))
 (segment (start 162.179 127.635) (end 163.449 126.365) (width 0.508) (layer B.Cu) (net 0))
 (segment (start 163.449 126.365) (end 164.846 126.365) (width 0.508) (layer B.Cu) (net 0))
 (segment (start 159.552 127.421) (end 161.29 129.159) (width 0.508) (layer B.Cu) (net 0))
 (segment (start 159.552 118.999) (end 159.552 127.421) (width 0.508) (layer B.Cu) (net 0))
 (segment (start 154.178 119.507) (end 159.004 119.507) (width 0.508) (layer B.Cu) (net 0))
 (segment (start 164.719 127.635) (end 166.624 127.635) (width 0.508) (layer B.Cu) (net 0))
 (segment (start 163.195 129.159) (end 164.719 127.635) (width 0.508) (layer B.Cu) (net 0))
 (segment (start 161.29 129.159) (end 163.195 129.159) (width 0.508) (layer B.Cu) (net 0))
 (segment (start 159.004 119.507) (end 159.512 118.999) (width 0.508) (layer B.Cu) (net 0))
 (segment (start 162.052 118.872) (end 162.306 118.872) (width 0.508) (layer B.Cu) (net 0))
 (segment (start 162.052 122.174) (end 162.052 118.872) (width 0.508) (layer B.Cu) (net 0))
 (segment (start 162.052 117.983) (end 162.052 118.999) (width 0.508) (layer B.Cu) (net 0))
 (segment (start 165.354 114.681) (end 165.354 113.538) (width 0.508) (layer B.Cu) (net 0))
 (segment (start 162.052 117.983) (end 165.354 114.681) (width 0.508) (layer B.Cu) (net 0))
 (segment (start 162.052 117.094) (end 162.052 117.983) (width 0.508) (layer B.Cu) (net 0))
 (segment (start 159.766 114.808) (end 162.052 117.094) (width 0.508) (layer B.Cu) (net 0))
 (segment (start 159.004 114.808) (end 159.766 114.808) (width 0.508) (layer B.Cu) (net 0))
 (segment (start 153.797 113.538) (end 156.845 113.538) (width 0.508) (layer B.Cu) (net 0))
 (segment (start 152.781 114.554) (end 153.797 113.538) (width 0.508) (layer B.Cu) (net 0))
 (segment (start 149.36363 114.554) (end 152.781 114.554) (width 0.508) (layer B.Cu) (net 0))
 (segment (start 147.828 113.01837) (end 149.36363 114.554) (width 0.508) (layer B.Cu) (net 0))
 (segment (start 147.828 111.887) (end 147.828 113.01837) (width 0.508) (layer B.Cu) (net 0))
 (segment (start 108.204 125.095) (end 107.569 125.095) (width 0.508) (layer B.Cu) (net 11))
 (segment (start 119.086 127.635) (end 121.539 127.635) (width 0.508) (layer B.Cu) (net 11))
 (segment (start 117.475 129.286) (end 119.126 127.635) (width 0.508) (layer B.Cu) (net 11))
 (segment (start 112.014 129.286) (end 117.475 129.286) (width 0.508) (layer B.Cu) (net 11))
 (segment (start 110.871 128.143) (end 112.014 129.286) (width 0.508) (layer B.Cu) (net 11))
 (segment (start 110.871 126.238) (end 110.871 128.143) (width 0.508) (layer B.Cu) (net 11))
 (segment (start 109.728 125.095) (end 110.871 126.238) (width 0.508) (layer B.Cu) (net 11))
 (segment (start 108.204 125.095) (end 109.728 125.095) (width 0.508) (layer B.Cu) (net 11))
 (segment (start 113.665 120.65) (end 114.808 119.507) (width 0.508) (layer B.Cu) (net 10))
 (segment (start 108.204 120.65) (end 109.728 120.65) (width 0.508) (layer B.Cu) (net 10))
 (segment (start 109.728 120.65) (end 110.363 121.285) (width 0.508) (layer B.Cu) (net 10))
 (segment (start 113.03 121.285) (end 113.665 120.65) (width 0.508) (layer B.Cu) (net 10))
 (segment (start 110.363 121.285) (end 113.03 121.285) (width 0.508) (layer B.Cu) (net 10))
 (segment (start 116.586 127.635) (end 119.126 125.095) (width 0.508) (layer B.Cu) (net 8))
 (segment (start 119.126 125.095) (end 119.126 123.317) (width 0.508) (layer B.Cu) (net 8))
 (segment (start 118.491 119.888) (end 118.11 119.507) (width 0.508) (layer B.Cu) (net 8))
 (segment (start 118.491 123.317) (end 118.491 119.888) (width 0.508) (layer B.Cu) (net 8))
 (segment (start 118.364 123.444) (end 118.491 123.317) (width 0.508) (layer B.Cu) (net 8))
 (segment (start 107.696 115.57) (end 108.204 115.57) (width 0.508) (layer B.Cu) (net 6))
 (segment (start 115.316 124.714) (end 116.459 124.714) (width 0.508) (layer B.Cu) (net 6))
 (segment (start 125.603 111.887) (end 121.158 111.887) (width 0.508) (layer B.Cu) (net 6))
 (segment (start 125.984 112.268) (end 125.603 111.887) (width 0.508) (layer B.Cu) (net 6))
 (segment (start 106.426 116.459) (end 106.426 121.92) (width 0.508) (layer B.Cu) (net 6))
 (segment (start 107.315 115.57) (end 106.426 116.459) (width 0.508) (layer B.Cu) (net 6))
 (segment (start 108.204 115.57) (end 107.315 115.57) (width 0.508) (layer B.Cu) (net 6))
 (segment (start 125.984 112.268) (end 126.746 112.268) (width 0.508) (layer B.Cu) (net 6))
 (segment (start 126.746 112.268) (end 129.286 114.808) (width 0.508) (layer B.Cu) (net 6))
 (segment (start 129.286 114.808) (end 130.175 114.808) (width 0.508) (layer B.Cu) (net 6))
 (segment (start 130.175 114.808) (end 130.302 114.808) (width 0.508) (layer B.Cu) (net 6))
 (segment (start 117.094 113.665) (end 119.253 113.665) (width 0.508) (layer B.Cu) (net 6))
 (segment (start 116.332 112.903) (end 117.094 113.665) (width 0.508) (layer B.Cu) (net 6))
 (segment (start 119.253 113.665) (end 121.158 111.76) (width 0.508) (layer B.Cu) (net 6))
 (segment (start 116.332 110.617) (end 116.332 112.903) (width 0.508) (layer B.Cu) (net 6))
 (segment (start 115.951 110.236) (end 116.332 110.617) (width 0.508) (layer B.Cu) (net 6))
 (segment (start 113.411 110.236) (end 115.951 110.236) (width 0.508) (layer B.Cu) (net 6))
 (segment (start 113.157 110.49) (end 113.411 110.236) (width 0.508) (layer B.Cu) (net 6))
 (segment (start 113.157 114.808) (end 113.157 110.49) (width 0.508) (layer B.Cu) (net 6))
 (segment (start 112.395 115.57) (end 113.157 114.808) (width 0.508) (layer B.Cu) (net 6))
 (segment (start 108.204 115.57) (end 112.395 115.57) (width 0.508) (layer B.Cu) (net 6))
 (segment (start 106.426 121.92) (end 106.426 127) (width 0.508) (layer B.Cu) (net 6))
 (segment (start 106.426 127) (end 107.061 127.635) (width 0.508) (layer B.Cu) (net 6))
 (segment (start 107.061 127.635) (end 108.331 127.635) (width 0.508) (layer B.Cu) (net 6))
 (segment (start 113.284 122.809) (end 115.189 124.714) (width 0.508) (layer B.Cu) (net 6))
 (segment (start 115.189 124.714) (end 117.094 124.714) (width 0.508) (layer B.Cu) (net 6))
 (segment (start 106.426 122.809) (end 113.284 122.809) (width 0.508) (layer B.Cu) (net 6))
 (segment (start 106.426 121.92) (end 106.426 122.809) (width 0.508) (layer B.Cu) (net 6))
 (segment (start 116.459 122.174) (end 117.094 122.174) (width 0.508) (layer B.Cu) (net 1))
 (segment (start 116.332 122.047) (end 116.459 122.174) (width 0.508) (layer B.Cu) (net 1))
 (segment (start 116.332 117.983) (end 116.332 122.047) (width 0.508) (layer B.Cu) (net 1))
 (segment (start 108.204 118.11) (end 108.331 117.983) (width 0.508) (layer B.Cu) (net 1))
 (segment (start 116.332 117.983) (end 119.507 117.983) (width 0.508) (layer B.Cu) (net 1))
 (segment (start 119.507 120.904) (end 119.507 117.983) (width 0.508) (layer B.Cu) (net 1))
 (segment (start 120.777 122.174) (end 119.507 120.904) (width 0.508) (layer B.Cu) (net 1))
 (segment (start 121.412 122.174) (end 120.777 122.174) (width 0.508) (layer B.Cu) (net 1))
 (segment (start 111.252 117.983) (end 108.331 117.983) (width 0.508) (layer B.Cu) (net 1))
 (segment (start 111.633 119.507) (end 111.633 117.983) (width 0.508) (layer B.Cu) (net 1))
 (segment (start 111.633 117.983) (end 116.332 117.983) (width 0.508) (layer B.Cu) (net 1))
 (segment (start 111.252 117.983) (end 111.633 117.983) (width 0.508) (layer B.Cu) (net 1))
 (segment (start 110.617 113.03) (end 111.633 112.014) (width 0.508) (layer B.Cu) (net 2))
 (segment (start 111.633 112.014) (end 111.633 111.887) (width 0.508) (layer B.Cu) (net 2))
 (segment (start 108.204 113.03) (end 110.617 113.03) (width 0.508) (layer B.Cu) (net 2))
 (segment (start 111.633 111.887) (end 111.633 111.76) (width 0.508) (layer B.Cu) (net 2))
 (segment (start 116.967 108.585) (end 117.475 109.093) (width 0.508) (layer B.Cu) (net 2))
 (segment (start 113.411 108.585) (end 116.967 108.585) (width 0.508) (layer B.Cu) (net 2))
 (segment (start 111.633 110.363) (end 113.411 108.585) (width 0.508) (layer B.Cu) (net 2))
 (segment (start 111.633 111.379) (end 111.633 110.363) (width 0.508) (layer B.Cu) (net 2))
 (segment (start 133.477 112.522) (end 133.477 124.206) (width 0.508) (layer B.Cu) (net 2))
 (segment (start 128.524 107.569) (end 133.477 112.522) (width 0.508) (layer B.Cu) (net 2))
 (segment (start 123.825 107.569) (end 128.524 107.569) (width 0.508) (layer B.Cu) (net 2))
 (segment (start 122.809 108.585) (end 123.825 107.569) (width 0.508) (layer B.Cu) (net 2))
 (segment (start 117.983 108.585) (end 122.809 108.585) (width 0.508) (layer B.Cu) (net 2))
 (segment (start 133.477 124.206) (end 134.366 125.095) (width 0.508) (layer B.Cu) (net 2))
 (segment (start 117.475 109.093) (end 117.983 108.585) (width 0.508) (layer B.Cu) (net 2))
 (segment (start 125.095 109.093) (end 126.111 109.093) (width 0.508) (layer B.Cu) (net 3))
 (segment (start 126.111 109.093) (end 129.286 112.268) (width 0.508) (layer B.Cu) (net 3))
 (segment (start 124.46 109.855) (end 125.222 109.093) (width 0.508) (layer B.Cu) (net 3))
 (segment (start 120.396 109.855) (end 124.46 109.855) (width 0.508) (layer B.Cu) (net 3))
 (segment (start 118.364 111.887) (end 120.396 109.855) (width 0.508) (layer B.Cu) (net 3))
 (segment (start 117.983 111.887) (end 118.364 111.887) (width 0.508) (layer B.Cu) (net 3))
 (segment (start 129.159 127.635) (end 130.429 126.365) (width 0.508) (layer B.Cu) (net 9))
 (segment (start 130.429 126.365) (end 131.826 126.365) (width 0.508) (layer B.Cu) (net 9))
 (segment (start 131.699 127.635) (end 133.604 127.635) (width 0.508) (layer B.Cu) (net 5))
 (segment (start 130.175 129.159) (end 131.699 127.635) (width 0.508) (layer B.Cu) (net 5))
 (segment (start 128.27 129.159) (end 130.175 129.159) (width 0.508) (layer B.Cu) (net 5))
 (segment (start 126.532 127.421) (end 128.27 129.159) (width 0.508) (layer B.Cu) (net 5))
 (segment (start 126.532 118.999) (end 126.532 127.421) (width 0.508) (layer B.Cu) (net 5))
 (segment (start 121.158 119.507) (end 125.984 119.507) (width 0.508) (layer B.Cu) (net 5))
 (segment (start 125.984 119.507) (end 126.492 118.999) (width 0.508) (layer B.Cu) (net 5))
 (segment (start 129.032 118.872) (end 129.286 118.872) (width 0.508) (layer B.Cu) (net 4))
 (segment (start 129.032 122.174) (end 129.032 118.872) (width 0.508) (layer B.Cu) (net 4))
 (segment (start 129.032 117.983) (end 129.032 118.999) (width 0.508) (layer B.Cu) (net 4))
 (segment (start 132.334 114.681) (end 132.334 113.538) (width 0.508) (layer B.Cu) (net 4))
 (segment (start 129.032 117.983) (end 132.334 114.681) (width 0.508) (layer B.Cu) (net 4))
 (segment (start 129.032 117.094) (end 129.032 117.983) (width 0.508) (layer B.Cu) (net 4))
 (segment (start 126.746 114.808) (end 129.032 117.094) (width 0.508) (layer B.Cu) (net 4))
 (segment (start 125.984 114.808) (end 126.746 114.808) (width 0.508) (layer B.Cu) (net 4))
 (segment (start 120.777 113.538) (end 123.825 113.538) (width 0.508) (layer B.Cu) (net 7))
 (segment (start 119.761 114.554) (end 120.777 113.538) (width 0.508) (layer B.Cu) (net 7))
 (segment (start 116.34363 114.554) (end 119.761 114.554) (width 0.508) (layer B.Cu) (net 7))
 (segment (start 114.808 113.01837) (end 116.34363 114.554) (width 0.508) (layer B.Cu) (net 7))
 (segment (start 114.808 111.887) (end 114.808 113.01837) (width 0.508) (layer B.Cu) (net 7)))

